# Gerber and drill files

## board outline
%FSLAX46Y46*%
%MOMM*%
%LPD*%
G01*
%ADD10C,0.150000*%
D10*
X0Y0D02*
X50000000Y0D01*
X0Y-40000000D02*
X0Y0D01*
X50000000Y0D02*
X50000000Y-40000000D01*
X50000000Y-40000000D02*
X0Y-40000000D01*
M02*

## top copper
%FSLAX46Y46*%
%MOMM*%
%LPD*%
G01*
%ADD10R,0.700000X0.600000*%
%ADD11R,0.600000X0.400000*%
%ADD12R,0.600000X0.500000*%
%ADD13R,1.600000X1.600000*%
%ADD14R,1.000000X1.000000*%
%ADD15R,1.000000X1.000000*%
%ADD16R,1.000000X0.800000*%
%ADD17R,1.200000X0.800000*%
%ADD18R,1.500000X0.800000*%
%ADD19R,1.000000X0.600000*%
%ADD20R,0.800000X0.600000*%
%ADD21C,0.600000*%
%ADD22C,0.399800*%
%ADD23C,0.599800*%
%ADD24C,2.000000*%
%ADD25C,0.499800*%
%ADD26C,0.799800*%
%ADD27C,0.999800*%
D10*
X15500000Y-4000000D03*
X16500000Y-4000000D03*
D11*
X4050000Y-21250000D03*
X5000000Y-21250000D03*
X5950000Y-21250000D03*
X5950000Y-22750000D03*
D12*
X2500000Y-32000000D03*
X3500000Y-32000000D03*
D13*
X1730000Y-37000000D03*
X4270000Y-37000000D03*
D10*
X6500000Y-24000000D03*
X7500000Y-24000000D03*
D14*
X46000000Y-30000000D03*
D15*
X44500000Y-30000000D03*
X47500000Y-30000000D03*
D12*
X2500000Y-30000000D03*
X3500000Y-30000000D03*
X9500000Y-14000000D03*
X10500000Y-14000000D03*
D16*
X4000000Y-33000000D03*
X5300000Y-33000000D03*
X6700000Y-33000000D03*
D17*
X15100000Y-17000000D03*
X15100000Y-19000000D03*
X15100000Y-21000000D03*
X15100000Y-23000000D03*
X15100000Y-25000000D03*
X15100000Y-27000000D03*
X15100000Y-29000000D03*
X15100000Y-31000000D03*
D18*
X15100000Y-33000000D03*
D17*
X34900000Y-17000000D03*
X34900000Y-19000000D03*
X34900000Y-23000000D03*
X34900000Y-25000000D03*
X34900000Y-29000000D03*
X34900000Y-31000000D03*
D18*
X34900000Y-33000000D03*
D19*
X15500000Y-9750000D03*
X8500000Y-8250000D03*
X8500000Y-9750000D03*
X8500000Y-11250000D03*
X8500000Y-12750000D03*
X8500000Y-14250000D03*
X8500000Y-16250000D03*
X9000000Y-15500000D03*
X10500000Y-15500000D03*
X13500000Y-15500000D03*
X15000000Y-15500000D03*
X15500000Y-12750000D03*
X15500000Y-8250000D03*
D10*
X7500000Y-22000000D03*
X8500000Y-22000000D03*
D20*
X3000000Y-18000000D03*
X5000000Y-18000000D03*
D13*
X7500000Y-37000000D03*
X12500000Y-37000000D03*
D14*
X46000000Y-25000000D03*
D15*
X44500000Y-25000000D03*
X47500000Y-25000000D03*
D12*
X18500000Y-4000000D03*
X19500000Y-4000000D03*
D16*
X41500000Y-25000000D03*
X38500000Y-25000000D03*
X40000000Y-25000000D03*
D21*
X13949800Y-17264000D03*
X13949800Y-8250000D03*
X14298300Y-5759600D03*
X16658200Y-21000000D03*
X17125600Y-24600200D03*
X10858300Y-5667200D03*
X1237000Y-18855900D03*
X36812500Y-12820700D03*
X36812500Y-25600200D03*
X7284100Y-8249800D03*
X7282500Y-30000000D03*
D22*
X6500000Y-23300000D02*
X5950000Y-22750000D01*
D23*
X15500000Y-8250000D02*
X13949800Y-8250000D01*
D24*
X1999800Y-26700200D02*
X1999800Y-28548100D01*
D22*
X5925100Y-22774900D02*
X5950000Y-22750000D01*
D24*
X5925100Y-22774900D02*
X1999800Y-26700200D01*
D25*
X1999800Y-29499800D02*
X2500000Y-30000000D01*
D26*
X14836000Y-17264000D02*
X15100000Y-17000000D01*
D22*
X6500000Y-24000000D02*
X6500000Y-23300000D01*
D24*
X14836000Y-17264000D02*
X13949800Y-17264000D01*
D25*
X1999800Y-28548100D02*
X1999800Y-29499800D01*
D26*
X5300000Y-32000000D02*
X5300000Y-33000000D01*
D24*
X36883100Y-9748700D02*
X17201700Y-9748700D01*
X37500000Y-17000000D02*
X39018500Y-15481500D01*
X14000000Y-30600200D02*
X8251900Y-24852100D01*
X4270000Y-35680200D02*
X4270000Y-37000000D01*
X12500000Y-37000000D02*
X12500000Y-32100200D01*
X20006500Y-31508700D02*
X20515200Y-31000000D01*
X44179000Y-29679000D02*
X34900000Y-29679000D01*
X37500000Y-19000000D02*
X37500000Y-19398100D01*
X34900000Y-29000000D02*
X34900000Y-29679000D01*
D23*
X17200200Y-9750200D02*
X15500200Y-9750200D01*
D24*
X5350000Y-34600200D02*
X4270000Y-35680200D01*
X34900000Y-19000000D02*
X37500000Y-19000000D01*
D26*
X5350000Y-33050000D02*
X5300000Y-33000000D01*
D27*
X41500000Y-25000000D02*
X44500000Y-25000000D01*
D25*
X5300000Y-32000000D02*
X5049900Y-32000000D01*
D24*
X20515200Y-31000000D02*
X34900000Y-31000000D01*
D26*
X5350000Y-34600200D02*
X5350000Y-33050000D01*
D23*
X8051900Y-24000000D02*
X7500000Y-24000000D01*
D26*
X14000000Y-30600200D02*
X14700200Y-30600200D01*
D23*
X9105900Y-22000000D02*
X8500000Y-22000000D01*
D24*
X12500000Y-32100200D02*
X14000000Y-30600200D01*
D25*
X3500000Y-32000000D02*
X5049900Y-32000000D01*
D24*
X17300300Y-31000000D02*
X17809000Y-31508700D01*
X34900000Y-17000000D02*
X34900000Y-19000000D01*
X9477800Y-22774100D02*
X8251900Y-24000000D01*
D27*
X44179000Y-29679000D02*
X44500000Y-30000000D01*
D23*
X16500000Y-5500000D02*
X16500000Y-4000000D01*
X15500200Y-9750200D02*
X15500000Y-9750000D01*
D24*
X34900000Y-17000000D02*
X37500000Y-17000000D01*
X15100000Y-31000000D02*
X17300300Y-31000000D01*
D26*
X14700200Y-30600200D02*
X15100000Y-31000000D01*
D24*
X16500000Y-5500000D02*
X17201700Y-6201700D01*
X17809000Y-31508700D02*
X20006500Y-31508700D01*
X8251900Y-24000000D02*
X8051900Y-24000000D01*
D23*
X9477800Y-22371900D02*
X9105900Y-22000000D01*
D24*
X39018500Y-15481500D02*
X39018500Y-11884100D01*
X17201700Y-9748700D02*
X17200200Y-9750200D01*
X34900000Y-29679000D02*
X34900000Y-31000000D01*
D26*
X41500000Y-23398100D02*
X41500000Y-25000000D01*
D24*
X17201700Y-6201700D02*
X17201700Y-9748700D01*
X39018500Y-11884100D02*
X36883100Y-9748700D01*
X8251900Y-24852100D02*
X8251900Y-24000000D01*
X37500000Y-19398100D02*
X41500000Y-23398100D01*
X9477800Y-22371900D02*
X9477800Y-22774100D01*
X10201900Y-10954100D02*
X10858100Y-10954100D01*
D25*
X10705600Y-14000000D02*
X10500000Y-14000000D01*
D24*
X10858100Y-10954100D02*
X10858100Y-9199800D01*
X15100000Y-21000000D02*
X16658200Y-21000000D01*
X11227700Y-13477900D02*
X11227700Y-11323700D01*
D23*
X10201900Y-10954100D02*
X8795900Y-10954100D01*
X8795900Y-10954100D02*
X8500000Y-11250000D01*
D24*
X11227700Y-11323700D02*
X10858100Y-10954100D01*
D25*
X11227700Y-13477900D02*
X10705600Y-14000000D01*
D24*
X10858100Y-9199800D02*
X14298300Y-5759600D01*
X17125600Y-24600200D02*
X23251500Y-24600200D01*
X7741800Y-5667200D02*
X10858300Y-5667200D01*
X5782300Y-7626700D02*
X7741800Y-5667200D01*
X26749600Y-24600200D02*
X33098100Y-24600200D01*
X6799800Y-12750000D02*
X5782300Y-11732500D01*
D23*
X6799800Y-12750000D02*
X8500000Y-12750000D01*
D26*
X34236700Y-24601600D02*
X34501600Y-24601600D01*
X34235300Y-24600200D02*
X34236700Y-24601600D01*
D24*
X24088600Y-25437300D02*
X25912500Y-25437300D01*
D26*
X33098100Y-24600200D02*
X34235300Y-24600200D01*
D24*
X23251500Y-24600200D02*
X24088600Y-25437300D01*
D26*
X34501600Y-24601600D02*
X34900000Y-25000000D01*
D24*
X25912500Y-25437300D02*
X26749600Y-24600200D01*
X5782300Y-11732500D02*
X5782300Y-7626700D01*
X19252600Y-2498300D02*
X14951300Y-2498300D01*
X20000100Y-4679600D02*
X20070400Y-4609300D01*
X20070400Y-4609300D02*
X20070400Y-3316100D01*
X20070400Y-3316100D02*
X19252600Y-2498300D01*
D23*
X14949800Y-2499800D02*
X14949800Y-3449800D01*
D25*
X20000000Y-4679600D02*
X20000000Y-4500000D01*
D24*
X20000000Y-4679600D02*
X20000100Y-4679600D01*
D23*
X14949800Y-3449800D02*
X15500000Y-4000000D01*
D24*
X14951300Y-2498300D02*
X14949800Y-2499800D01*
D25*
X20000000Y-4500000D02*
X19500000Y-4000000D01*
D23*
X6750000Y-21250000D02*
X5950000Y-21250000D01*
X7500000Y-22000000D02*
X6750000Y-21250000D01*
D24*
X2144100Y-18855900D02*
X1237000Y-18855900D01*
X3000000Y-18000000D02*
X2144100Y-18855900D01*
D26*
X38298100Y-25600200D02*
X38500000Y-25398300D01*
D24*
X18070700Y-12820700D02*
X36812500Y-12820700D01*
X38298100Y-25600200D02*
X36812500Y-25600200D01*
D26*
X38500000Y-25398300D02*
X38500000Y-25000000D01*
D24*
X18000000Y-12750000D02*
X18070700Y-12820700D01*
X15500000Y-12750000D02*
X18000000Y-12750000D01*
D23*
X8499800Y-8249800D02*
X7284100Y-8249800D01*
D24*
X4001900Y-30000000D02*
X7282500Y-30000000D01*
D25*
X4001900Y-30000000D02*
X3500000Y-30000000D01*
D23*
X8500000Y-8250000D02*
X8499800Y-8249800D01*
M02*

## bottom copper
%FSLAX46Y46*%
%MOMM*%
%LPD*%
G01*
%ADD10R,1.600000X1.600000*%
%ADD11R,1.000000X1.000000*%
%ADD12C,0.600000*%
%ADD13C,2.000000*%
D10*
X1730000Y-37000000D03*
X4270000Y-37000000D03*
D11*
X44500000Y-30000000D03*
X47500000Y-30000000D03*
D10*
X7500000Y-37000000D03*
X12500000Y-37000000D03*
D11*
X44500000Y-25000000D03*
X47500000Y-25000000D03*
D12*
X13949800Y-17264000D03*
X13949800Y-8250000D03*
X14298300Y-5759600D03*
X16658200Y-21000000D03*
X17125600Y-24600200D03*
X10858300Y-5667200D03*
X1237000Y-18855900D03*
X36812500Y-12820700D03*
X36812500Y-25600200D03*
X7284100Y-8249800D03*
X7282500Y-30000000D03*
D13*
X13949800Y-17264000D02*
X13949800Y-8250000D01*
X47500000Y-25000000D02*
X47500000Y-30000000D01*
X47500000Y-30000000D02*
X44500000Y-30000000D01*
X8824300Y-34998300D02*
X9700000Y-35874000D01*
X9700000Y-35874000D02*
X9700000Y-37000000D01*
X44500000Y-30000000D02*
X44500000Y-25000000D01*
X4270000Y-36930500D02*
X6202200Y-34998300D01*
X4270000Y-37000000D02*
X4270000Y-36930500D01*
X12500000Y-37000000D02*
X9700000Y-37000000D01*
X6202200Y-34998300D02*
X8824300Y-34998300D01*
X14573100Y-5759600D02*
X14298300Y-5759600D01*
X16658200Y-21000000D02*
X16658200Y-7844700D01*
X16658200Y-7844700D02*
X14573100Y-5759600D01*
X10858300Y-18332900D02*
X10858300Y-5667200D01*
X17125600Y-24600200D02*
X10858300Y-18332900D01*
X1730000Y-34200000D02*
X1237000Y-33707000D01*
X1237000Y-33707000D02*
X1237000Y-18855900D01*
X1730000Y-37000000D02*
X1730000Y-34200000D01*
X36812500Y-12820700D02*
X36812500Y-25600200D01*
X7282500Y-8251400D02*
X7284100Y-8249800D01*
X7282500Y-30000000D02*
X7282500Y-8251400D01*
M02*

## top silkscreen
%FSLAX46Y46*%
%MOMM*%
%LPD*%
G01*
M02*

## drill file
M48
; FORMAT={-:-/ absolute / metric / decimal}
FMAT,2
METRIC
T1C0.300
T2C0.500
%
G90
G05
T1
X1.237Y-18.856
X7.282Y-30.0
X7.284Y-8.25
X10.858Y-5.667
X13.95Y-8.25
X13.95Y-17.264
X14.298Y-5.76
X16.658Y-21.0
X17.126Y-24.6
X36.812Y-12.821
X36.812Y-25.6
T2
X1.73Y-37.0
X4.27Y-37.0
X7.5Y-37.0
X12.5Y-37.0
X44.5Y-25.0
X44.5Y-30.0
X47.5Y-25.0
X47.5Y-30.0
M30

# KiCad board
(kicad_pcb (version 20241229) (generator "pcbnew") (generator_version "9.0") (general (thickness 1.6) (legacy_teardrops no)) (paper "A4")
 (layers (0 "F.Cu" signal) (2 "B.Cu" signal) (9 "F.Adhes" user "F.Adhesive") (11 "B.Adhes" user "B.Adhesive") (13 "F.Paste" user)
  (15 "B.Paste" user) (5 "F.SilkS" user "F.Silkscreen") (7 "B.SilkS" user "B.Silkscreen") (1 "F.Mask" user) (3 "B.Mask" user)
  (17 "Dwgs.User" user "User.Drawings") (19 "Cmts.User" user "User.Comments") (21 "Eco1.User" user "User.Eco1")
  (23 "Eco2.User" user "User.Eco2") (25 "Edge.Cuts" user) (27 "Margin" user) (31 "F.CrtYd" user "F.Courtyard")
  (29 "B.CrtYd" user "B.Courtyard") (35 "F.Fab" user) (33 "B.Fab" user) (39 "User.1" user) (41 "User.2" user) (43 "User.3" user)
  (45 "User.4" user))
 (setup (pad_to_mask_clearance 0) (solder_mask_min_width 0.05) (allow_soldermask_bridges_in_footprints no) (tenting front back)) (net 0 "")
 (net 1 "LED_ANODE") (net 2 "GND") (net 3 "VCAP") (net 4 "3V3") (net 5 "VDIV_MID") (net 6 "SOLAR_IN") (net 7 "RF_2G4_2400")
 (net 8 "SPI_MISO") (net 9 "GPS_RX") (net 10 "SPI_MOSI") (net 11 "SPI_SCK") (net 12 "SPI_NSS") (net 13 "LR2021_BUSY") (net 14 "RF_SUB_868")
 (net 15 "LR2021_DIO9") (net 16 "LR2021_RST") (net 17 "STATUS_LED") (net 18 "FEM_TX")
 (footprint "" (layer "F.Cu") (at 16 4)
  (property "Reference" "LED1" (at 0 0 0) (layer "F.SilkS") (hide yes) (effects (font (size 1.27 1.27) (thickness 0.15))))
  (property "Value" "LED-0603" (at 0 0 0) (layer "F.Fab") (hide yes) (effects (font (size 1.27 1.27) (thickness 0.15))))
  (pad "A" smd rect (at -0.5 0) (size 0.7 0.6) (layers "F.Cu" "F.Mask") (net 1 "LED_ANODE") (thermal_bridge_angle 45))
  (pad "K" smd rect (at 0.5 0) (size 0.7 0.6) (layers "F.Cu" "F.Mask") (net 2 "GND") (thermal_bridge_angle 45)))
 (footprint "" (layer "F.Cu") (at 5 22)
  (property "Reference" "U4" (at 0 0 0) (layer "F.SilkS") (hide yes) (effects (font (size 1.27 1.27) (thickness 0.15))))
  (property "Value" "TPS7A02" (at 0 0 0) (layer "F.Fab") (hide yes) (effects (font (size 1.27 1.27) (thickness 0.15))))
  (pad "1" smd rect (at -0.95 -0.75) (size 0.6 0.4) (layers "F.Cu" "F.Mask") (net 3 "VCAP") (thermal_bridge_angle 45))
  (pad "2" smd rect (at 0 -0.75) (size 0.6 0.4) (layers "F.Cu" "F.Mask") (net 2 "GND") (thermal_bridge_angle 45))
  (pad "3" smd rect (at 0.95 -0.75) (size 0.6 0.4) (layers "F.Cu" "F.Mask") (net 3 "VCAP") (thermal_bridge_angle 45))
  (pad "4" smd rect (at 0.95 0.75) (size 0.6 0.4) (layers "F.Cu" "F.Mask") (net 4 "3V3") (thermal_bridge_angle 45)))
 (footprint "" (layer "F.Cu") (at 3 32)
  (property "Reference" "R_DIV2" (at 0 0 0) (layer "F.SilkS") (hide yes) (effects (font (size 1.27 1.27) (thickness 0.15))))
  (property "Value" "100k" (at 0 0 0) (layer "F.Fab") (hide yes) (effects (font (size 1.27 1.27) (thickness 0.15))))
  (pad "1" smd rect (at -0.5 0) (size 0.6 0.5) (layers "F.Cu" "F.Mask") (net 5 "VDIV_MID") (thermal_bridge_angle 45))
  (pad "2" smd rect (at 0.5 0) (size 0.6 0.5) (layers "F.Cu" "F.Mask") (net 2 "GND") (thermal_bridge_angle 45)))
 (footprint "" (layer "F.Cu") (at 3 37)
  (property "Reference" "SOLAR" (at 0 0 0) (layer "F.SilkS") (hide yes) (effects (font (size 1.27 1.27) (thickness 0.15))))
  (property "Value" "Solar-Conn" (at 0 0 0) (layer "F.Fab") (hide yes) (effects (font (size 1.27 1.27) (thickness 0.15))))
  (pad "1" thru_hole rect (at -1.27 0) (size 1.6 1.6) (drill 0.5) (layers "*.Cu" "*.Mask") (remove_unused_layers no) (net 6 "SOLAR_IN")
   (thermal_bridge_angle 45))
  (pad "2" thru_hole rect (at 1.27 0) (size 1.6 1.6) (drill 0.5) (layers "*.Cu" "*.Mask") (remove_unused_layers no) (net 2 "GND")
   (thermal_bridge_angle 45)))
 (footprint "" (layer "F.Cu") (at 7 24)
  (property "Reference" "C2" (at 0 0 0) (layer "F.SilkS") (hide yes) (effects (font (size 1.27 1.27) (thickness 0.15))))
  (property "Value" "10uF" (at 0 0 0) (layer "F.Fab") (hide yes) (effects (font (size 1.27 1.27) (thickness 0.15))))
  (pad "1" smd rect (at -0.5 0) (size 0.7 0.6) (layers "F.Cu" "F.Mask") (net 4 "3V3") (thermal_bridge_angle 45))
  (pad "2" smd rect (at 0.5 0) (size 0.7 0.6) (layers "F.Cu" "F.Mask") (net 2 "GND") (thermal_bridge_angle 45)))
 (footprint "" (layer "F.Cu") (at 46 30)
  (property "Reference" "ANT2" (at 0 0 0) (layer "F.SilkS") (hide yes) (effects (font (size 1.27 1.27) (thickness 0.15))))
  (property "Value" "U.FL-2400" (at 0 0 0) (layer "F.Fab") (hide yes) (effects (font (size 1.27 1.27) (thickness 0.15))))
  (pad "1" smd rect (at 0 0) (size 1 1) (layers "F.Cu" "F.Mask") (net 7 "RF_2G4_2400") (thermal_bridge_angle 45))
  (pad "2" thru_hole rect (at -1.5 0) (size 1 1) (drill 0.5) (layers "*.Cu" "*.Mask") (remove_unused_layers no) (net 2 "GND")
   (thermal_bridge_angle 45))
  (pad "3" thru_hole rect (at 1.5 0) (size 1 1) (drill 0.5) (layers "*.Cu" "*.Mask") (remove_unused_layers no) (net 2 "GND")
   (thermal_bridge_angle 45)))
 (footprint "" (layer "F.Cu") (at 3 30)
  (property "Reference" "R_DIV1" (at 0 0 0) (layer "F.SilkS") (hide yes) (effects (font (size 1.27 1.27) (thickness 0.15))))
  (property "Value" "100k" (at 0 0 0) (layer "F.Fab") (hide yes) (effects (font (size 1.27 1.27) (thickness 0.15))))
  (pad "1" smd rect (at -0.5 0) (size 0.6 0.5) (layers "F.Cu" "F.Mask") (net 4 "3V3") (thermal_bridge_angle 45))
  (pad "2" smd rect (at 0.5 0) (size 0.6 0.5) (layers "F.Cu" "F.Mask") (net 5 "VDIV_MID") (thermal_bridge_angle 45)))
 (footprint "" (layer "F.Cu") (at 10 14)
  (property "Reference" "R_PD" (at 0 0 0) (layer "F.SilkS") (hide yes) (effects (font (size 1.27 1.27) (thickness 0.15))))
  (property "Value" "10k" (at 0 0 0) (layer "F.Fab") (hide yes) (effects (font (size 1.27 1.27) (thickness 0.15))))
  (pad "1" smd rect (at -0.5 0) (size 0.6 0.5) (layers "F.Cu" "F.Mask") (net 2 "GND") (thermal_bridge_angle 45))
  (pad "2" smd rect (at 0.5 0) (size 0.6 0.5) (layers "F.Cu" "F.Mask") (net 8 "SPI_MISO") (thermal_bridge_angle 45)))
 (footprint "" (layer "F.Cu") (at 6 33)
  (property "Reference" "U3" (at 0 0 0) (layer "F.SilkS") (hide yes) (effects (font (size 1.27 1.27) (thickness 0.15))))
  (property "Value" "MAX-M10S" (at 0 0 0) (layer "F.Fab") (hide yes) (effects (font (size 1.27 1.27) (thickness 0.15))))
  (pad "1" smd rect (at -2 0) (size 1 0.8) (layers "F.Cu" "F.Mask") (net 4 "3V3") (thermal_bridge_angle 45))
  (pad "2" smd rect (at -0.7 0) (size 1 0.8) (layers "F.Cu" "F.Mask") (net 2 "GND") (thermal_bridge_angle 45))
  (pad "3" smd rect (at 0.7 0) (size 1 0.8) (layers "F.Cu" "F.Mask") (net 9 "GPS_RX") (thermal_bridge_angle 45)))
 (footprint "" (layer "F.Cu") (at 25 25)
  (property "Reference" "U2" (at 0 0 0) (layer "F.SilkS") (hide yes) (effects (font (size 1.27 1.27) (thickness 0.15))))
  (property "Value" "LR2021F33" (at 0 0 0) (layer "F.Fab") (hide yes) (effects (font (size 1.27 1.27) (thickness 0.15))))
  (pad "1" smd rect (at -9.9 -8) (size 1.2 0.8) (layers "F.Cu" "F.Mask") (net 4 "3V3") (thermal_bridge_angle 45))
  (pad "2" smd rect (at -9.9 -6) (size 1.2 0.8) (layers "F.Cu" "F.Mask") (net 2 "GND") (thermal_bridge_angle 45))
  (pad "3" smd rect (at -9.9 -4) (size 1.2 0.8) (layers "F.Cu" "F.Mask") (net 8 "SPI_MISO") (thermal_bridge_angle 45))
  (pad "4" smd rect (at -9.9 -2) (size 1.2 0.8) (layers "F.Cu" "F.Mask") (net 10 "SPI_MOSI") (thermal_bridge_angle 45))
  (pad "5" smd rect (at -9.9 0) (size 1.2 0.8) (layers "F.Cu" "F.Mask") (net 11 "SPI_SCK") (thermal_bridge_angle 45))
  (pad "6" smd rect (at -9.9 2) (size 1.2 0.8) (layers "F.Cu" "F.Mask") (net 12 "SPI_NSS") (thermal_bridge_angle 45))
  (pad "7" smd rect (at -9.9 4) (size 1.2 0.8) (layers "F.Cu" "F.Mask") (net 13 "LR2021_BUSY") (thermal_bridge_angle 45))
  (pad "8" smd rect (at -9.9 6) (size 1.2 0.8) (layers "F.Cu" "F.Mask") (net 2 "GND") (thermal_bridge_angle 45))
  (pad "9" smd rect (at -9.9 8) (size 1.5 0.8) (layers "F.Cu" "F.Mask") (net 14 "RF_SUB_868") (thermal_bridge_angle 45))
  (pad "10" smd rect (at 9.9 -8) (size 1.2 0.8) (layers "F.Cu" "F.Mask") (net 2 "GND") (thermal_bridge_angle 45))
  (pad "11" smd rect (at 9.9 -6) (size 1.2 0.8) (layers "F.Cu" "F.Mask") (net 2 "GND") (thermal_bridge_angle 45))
  (pad "13" smd rect (at 9.9 -2) (size 1.2 0.8) (layers "F.Cu" "F.Mask") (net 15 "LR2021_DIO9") (thermal_bridge_angle 45))
  (pad "14" smd rect (at 9.9 0) (size 1.2 0.8) (layers "F.Cu" "F.Mask") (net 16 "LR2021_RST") (thermal_bridge_angle 45))
  (pad "16" smd rect (at 9.9 4) (size 1.2 0.8) (layers "F.Cu" "F.Mask") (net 2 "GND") (thermal_bridge_angle 45))
  (pad "17" smd rect (at 9.9 6) (size 1.2 0.8) (layers "F.Cu" "F.Mask") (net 2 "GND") (thermal_bridge_angle 45))
  (pad "18" smd rect (at 9.9 8) (size 1.5 0.8) (layers "F.Cu" "F.Mask") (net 7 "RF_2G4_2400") (thermal_bridge_angle 45)))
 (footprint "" (layer "F.Cu") (at 12 12)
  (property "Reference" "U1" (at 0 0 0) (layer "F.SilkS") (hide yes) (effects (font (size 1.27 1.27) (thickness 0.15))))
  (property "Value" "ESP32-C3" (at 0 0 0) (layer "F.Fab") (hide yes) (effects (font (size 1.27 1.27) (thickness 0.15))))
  (pad "GND" smd rect (at 3.5 -2.25) (size 1 0.6) (layers "F.Cu" "F.Mask") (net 2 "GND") (thermal_bridge_angle 45))
  (pad "GPIO0" smd rect (at -3.5 -3.75) (size 1 0.6) (layers "F.Cu" "F.Mask") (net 5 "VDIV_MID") (thermal_bridge_angle 45))
  (pad "GPIO1" smd rect (at -3.5 -2.25) (size 1 0.6) (layers "F.Cu" "F.Mask") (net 9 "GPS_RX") (thermal_bridge_angle 45))
  (pad "GPIO2" smd rect (at -3.5 -0.75) (size 1 0.6) (layers "F.Cu" "F.Mask") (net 8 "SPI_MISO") (thermal_bridge_angle 45))
  (pad "GPIO3" smd rect (at -3.5 0.75) (size 1 0.6) (layers "F.Cu" "F.Mask") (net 16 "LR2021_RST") (thermal_bridge_angle 45))
  (pad "GPIO4" smd rect (at -3.5 2.25) (size 1 0.6) (layers "F.Cu" "F.Mask") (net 13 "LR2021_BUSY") (thermal_bridge_angle 45))
  (pad "GPIO5" smd rect (at -3.5 4.25) (size 1 0.6) (layers "F.Cu" "F.Mask") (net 15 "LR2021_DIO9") (thermal_bridge_angle 45))
  (pad "GPIO6" smd rect (at -3 3.5) (size 1 0.6) (layers "F.Cu" "F.Mask") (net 11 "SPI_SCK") (thermal_bridge_angle 45))
  (pad "GPIO7" smd rect (at -1.5 3.5) (size 1 0.6) (layers "F.Cu" "F.Mask") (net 10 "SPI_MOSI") (thermal_bridge_angle 45))
  (pad "GPIO9" smd rect (at 1.5 3.5) (size 1 0.6) (layers "F.Cu" "F.Mask") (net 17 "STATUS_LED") (thermal_bridge_angle 45))
  (pad "GPIO10" smd rect (at 3 3.5) (size 1 0.6) (layers "F.Cu" "F.Mask") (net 12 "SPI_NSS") (thermal_bridge_angle 45))
  (pad "GPIO19" smd rect (at 3.5 0.75) (size 1 0.6) (layers "F.Cu" "F.Mask") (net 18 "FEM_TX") (thermal_bridge_angle 45))
  (pad "VCC" smd rect (at 3.5 -3.75) (size 1 0.6) (layers "F.Cu" "F.Mask") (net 4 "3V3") (thermal_bridge_angle 45)))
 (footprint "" (layer "F.Cu") (at 8 22)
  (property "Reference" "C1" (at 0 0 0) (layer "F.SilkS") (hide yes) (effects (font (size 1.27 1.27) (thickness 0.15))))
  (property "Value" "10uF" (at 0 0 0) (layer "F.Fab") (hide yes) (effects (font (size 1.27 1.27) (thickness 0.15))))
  (pad "1" smd rect (at -0.5 0) (size 0.7 0.6) (layers "F.Cu" "F.Mask") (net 3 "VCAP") (thermal_bridge_angle 45))
  (pad "2" smd rect (at 0.5 0) (size 0.7 0.6) (layers "F.Cu" "F.Mask") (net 2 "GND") (thermal_bridge_angle 45)))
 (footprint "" (layer "F.Cu") (at 4 18)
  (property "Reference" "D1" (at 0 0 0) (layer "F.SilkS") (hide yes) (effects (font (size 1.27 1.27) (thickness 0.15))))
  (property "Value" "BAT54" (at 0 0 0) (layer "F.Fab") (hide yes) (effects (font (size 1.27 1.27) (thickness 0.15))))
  (pad "A" smd rect (at -1 0) (size 0.8 0.6) (layers "F.Cu" "F.Mask") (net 6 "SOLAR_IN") (thermal_bridge_angle 45))
  (pad "K" smd rect (at 1 0) (size 0.8 0.6) (layers "F.Cu" "F.Mask") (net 3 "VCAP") (thermal_bridge_angle 45)))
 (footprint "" (layer "F.Cu") (at 10 37)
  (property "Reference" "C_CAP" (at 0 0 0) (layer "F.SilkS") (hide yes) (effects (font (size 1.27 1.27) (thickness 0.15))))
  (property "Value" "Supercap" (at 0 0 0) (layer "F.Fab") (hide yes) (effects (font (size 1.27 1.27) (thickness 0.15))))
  (pad "1" thru_hole rect (at -2.5 0) (size 1.6 1.6) (drill 0.5) (layers "*.Cu" "*.Mask") (remove_unused_layers no) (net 3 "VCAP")
   (thermal_bridge_angle 45))
  (pad "2" thru_hole rect (at 2.5 0) (size 1.6 1.6) (drill 0.5) (layers "*.Cu" "*.Mask") (remove_unused_layers no) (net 2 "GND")
   (thermal_bridge_angle 45)))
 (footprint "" (layer "F.Cu") (at 46 25)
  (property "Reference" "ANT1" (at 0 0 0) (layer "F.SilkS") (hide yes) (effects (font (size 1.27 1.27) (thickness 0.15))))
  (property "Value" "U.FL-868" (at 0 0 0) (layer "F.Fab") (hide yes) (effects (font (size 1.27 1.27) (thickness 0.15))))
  (pad "1" smd rect (at 0 0) (size 1 1) (layers "F.Cu" "F.Mask") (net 14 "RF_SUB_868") (thermal_bridge_angle 45))
  (pad "2" thru_hole rect (at -1.5 0) (size 1 1) (drill 0.5) (layers "*.Cu" "*.Mask") (remove_unused_layers no) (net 2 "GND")
   (thermal_bridge_angle 45))
  (pad "3" thru_hole rect (at 1.5 0) (size 1 1) (drill 0.5) (layers "*.Cu" "*.Mask") (remove_unused_layers no) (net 2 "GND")
   (thermal_bridge_angle 45)))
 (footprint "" (layer "F.Cu") (at 19 4)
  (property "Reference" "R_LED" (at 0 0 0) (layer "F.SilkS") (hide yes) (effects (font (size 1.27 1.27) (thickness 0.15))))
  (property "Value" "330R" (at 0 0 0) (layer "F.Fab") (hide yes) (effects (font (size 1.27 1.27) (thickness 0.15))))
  (pad "1" smd rect (at -0.5 0) (size 0.6 0.5) (layers "F.Cu" "F.Mask") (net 17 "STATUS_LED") (thermal_bridge_angle 45))
  (pad "2" smd rect (at 0.5 0) (size 0.6 0.5) (layers "F.Cu" "F.Mask") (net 1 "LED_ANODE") (thermal_bridge_angle 45)))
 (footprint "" (layer "F.Cu") (at 40 25)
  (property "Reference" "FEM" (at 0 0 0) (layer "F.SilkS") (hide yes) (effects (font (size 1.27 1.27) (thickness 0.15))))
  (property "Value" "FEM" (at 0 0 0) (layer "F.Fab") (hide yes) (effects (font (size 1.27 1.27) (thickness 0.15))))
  (pad "GND" smd rect (at 1.5 0) (size 1 0.8) (layers "F.Cu" "F.Mask") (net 2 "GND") (thermal_bridge_angle 45))
  (pad "TX" smd rect (at -1.5 0) (size 1 0.8) (layers "F.Cu" "F.Mask") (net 18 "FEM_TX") (thermal_bridge_angle 45))
  (pad "VCC" smd rect (at 0 0) (size 1 0.8) (layers "F.Cu" "F.Mask") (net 4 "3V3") (thermal_bridge_angle 45)))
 (gr_line (start 0 0) (end 50 0) (stroke (width 0.15) (type default)) (layer "Edge.Cuts"))
 (gr_line (start 0 40) (end 0 0) (stroke (width 0.15) (type default)) (layer "Edge.Cuts"))
 (gr_line (start 50 0) (end 50 40) (stroke (width 0.15) (type default)) (layer "Edge.Cuts"))
 (gr_line (start 50 40) (end 0 40) (stroke (width 0.15) (type default)) (layer "Edge.Cuts"))
 (segment (start 6.5 23.3) (end 5.95 22.75) (width 0.3998) (layer "F.Cu") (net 4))
 (segment (start 15.5 8.25) (end 13.9498 8.25) (width 0.5998) (layer "F.Cu") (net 4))
 (segment (start 1.9998 26.7002) (end 1.9998 28.5481) (width 2) (layer "F.Cu") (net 4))
 (segment (start 5.9251 22.7749) (end 5.95 22.75) (width 0.3998) (layer "F.Cu") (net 4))
 (segment (start 5.9251 22.7749) (end 1.9998 26.7002) (width 2) (layer "F.Cu") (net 4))
 (segment (start 1.9998 29.4998) (end 2.5 30) (width 0.4998) (layer "F.Cu") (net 4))
 (segment (start 14.836 17.264) (end 15.1 17) (width 0.7998) (layer "F.Cu") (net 4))
 (segment (start 6.5 24) (end 6.5 23.3) (width 0.3998) (layer "F.Cu") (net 4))
 (segment (start 14.836 17.264) (end 13.9498 17.264) (width 2) (layer "F.Cu") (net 4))
 (segment (start 1.9998 28.5481) (end 1.9998 29.4998) (width 0.4998) (layer "F.Cu") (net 4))
 (via (at 13.9498 17.264) (size 0.6) (drill 0.3) (layers "F.Cu" "B.Cu") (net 4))
 (via (at 13.9498 8.25) (size 0.6) (drill 0.3) (layers "F.Cu" "B.Cu") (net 4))
 (segment (start 13.9498 17.264) (end 13.9498 8.25) (width 2) (layer "B.Cu") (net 4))
 (segment (start 5.3 32) (end 5.3 33) (width 0.7998) (layer "F.Cu") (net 2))
 (segment (start 36.8831 9.7487) (end 17.2017 9.7487) (width 2) (layer "F.Cu") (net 2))
 (segment (start 37.5 17) (end 39.0185 15.4815) (width 2) (layer "F.Cu") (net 2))
 (segment (start 14 30.6002) (end 8.2519 24.8521) (width 2) (layer "F.Cu") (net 2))
 (segment (start 4.27 35.6802) (end 4.27 37) (width 2) (layer "F.Cu") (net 2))
 (segment (start 12.5 37) (end 12.5 32.1002) (width 2) (layer "F.Cu") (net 2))
 (segment (start 20.0065 31.5087) (end 20.5152 31) (width 2) (layer "F.Cu") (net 2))
 (segment (start 44.179 29.679) (end 34.9 29.679) (width 2) (layer "F.Cu") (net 2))
 (segment (start 37.5 19) (end 37.5 19.3981) (width 2) (layer "F.Cu") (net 2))
 (segment (start 34.9 29) (end 34.9 29.679) (width 2) (layer "F.Cu") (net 2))
 (segment (start 17.2002 9.7502) (end 15.5002 9.7502) (width 0.5998) (layer "F.Cu") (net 2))
 (segment (start 5.35 34.6002) (end 4.27 35.6802) (width 2) (layer "F.Cu") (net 2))
 (segment (start 34.9 19) (end 37.5 19) (width 2) (layer "F.Cu") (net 2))
 (segment (start 5.35 33.05) (end 5.3 33) (width 0.7998) (layer "F.Cu") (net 2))
 (segment (start 41.5 25) (end 44.5 25) (width 0.9998) (layer "F.Cu") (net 2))
 (segment (start 5.3 32) (end 5.0499 32) (width 0.4998) (layer "F.Cu") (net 2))
 (segment (start 20.5152 31) (end 34.9 31) (width 2) (layer "F.Cu") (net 2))
 (segment (start 5.35 34.6002) (end 5.35 33.05) (width 0.7998) (layer "F.Cu") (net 2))
 (segment (start 8.0519 24) (end 7.5 24) (width 0.5998) (layer "F.Cu") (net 2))
 (segment (start 14 30.6002) (end 14.7002 30.6002) (width 0.7998) (layer "F.Cu") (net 2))
 (segment (start 9.1059 22) (end 8.5 22) (width 0.5998) (layer "F.Cu") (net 2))
 (segment (start 12.5 32.1002) (end 14 30.6002) (width 2) (layer "F.Cu") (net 2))
 (segment (start 3.5 32) (end 5.0499 32) (width 0.4998) (layer "F.Cu") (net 2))
 (segment (start 17.3003 31) (end 17.809 31.5087) (width 2) (layer "F.Cu") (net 2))
 (segment (start 34.9 17) (end 34.9 19) (width 2) (layer "F.Cu") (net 2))
 (segment (start 9.4778 22.7741) (end 8.2519 24) (width 2) (layer "F.Cu") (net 2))
 (segment (start 44.179 29.679) (end 44.5 30) (width 0.9998) (layer "F.Cu") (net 2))
 (segment (start 16.5 5.5) (end 16.5 4) (width 0.5998) (layer "F.Cu") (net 2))
 (segment (start 15.5002 9.7502) (end 15.5 9.75) (width 0.5998) (layer "F.Cu") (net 2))
 (segment (start 34.9 17) (end 37.5 17) (width 2) (layer "F.Cu") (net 2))
 (segment (start 15.1 31) (end 17.3003 31) (width 2) (layer "F.Cu") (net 2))
 (segment (start 14.7002 30.6002) (end 15.1 31) (width 0.7998) (layer "F.Cu") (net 2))
 (segment (start 16.5 5.5) (end 17.2017 6.2017) (width 2) (layer "F.Cu") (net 2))
 (segment (start 17.809 31.5087) (end 20.0065 31.5087) (width 2) (layer "F.Cu") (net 2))
 (segment (start 8.2519 24) (end 8.0519 24) (width 2) (layer "F.Cu") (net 2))
 (segment (start 9.4778 22.3719) (end 9.1059 22) (width 0.5998) (layer "F.Cu") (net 2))
 (segment (start 39.0185 15.4815) (end 39.0185 11.8841) (width 2) (layer "F.Cu") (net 2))
 (segment (start 17.2017 9.7487) (end 17.2002 9.7502) (width 2) (layer "F.Cu") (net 2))
 (segment (start 34.9 29.679) (end 34.9 31) (width 2) (layer "F.Cu") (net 2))
 (segment (start 41.5 23.3981) (end 41.5 25) (width 0.7998) (layer "F.Cu") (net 2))
 (segment (start 17.2017 6.2017) (end 17.2017 9.7487) (width 2) (layer "F.Cu") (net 2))
 (segment (start 39.0185 11.8841) (end 36.8831 9.7487) (width 2) (layer "F.Cu") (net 2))
 (segment (start 8.2519 24.8521) (end 8.2519 24) (width 2) (layer "F.Cu") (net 2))
 (segment (start 37.5 19.3981) (end 41.5 23.3981) (width 2) (layer "F.Cu") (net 2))
 (segment (start 9.4778 22.3719) (end 9.4778 22.7741) (width 2) (layer "F.Cu") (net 2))
 (segment (start 47.5 25) (end 47.5 30) (width 2) (layer "B.Cu") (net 2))
 (segment (start 47.5 30) (end 44.5 30) (width 2) (layer "B.Cu") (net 2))
 (segment (start 8.8243 34.9983) (end 9.7 35.874) (width 2) (layer "B.Cu") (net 2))
 (segment (start 9.7 35.874) (end 9.7 37) (width 2) (layer "B.Cu") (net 2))
 (segment (start 44.5 30) (end 44.5 25) (width 2) (layer "B.Cu") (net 2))
 (segment (start 4.27 36.9305) (end 6.2022 34.9983) (width 2) (layer "B.Cu") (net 2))
 (segment (start 4.27 37) (end 4.27 36.9305) (width 2) (layer "B.Cu") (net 2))
 (segment (start 12.5 37) (end 9.7 37) (width 2) (layer "B.Cu") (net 2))
 (segment (start 6.2022 34.9983) (end 8.8243 34.9983) (width 2) (layer "B.Cu") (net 2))
 (segment (start 10.2019 10.9541) (end 10.8581 10.9541) (width 2) (layer "F.Cu") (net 8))
 (segment (start 10.7056 14) (end 10.5 14) (width 0.4998) (layer "F.Cu") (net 8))
 (segment (start 10.8581 10.9541) (end 10.8581 9.1998) (width 2) (layer "F.Cu") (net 8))
 (segment (start 15.1 21) (end 16.6582 21) (width 2) (layer "F.Cu") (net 8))
 (segment (start 11.2277 13.4779) (end 11.2277 11.3237) (width 2) (layer "F.Cu") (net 8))
 (segment (start 10.2019 10.9541) (end 8.7959 10.9541) (width 0.5998) (layer "F.Cu") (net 8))
 (segment (start 8.7959 10.9541) (end 8.5 11.25) (width 0.5998) (layer "F.Cu") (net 8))
 (segment (start 11.2277 11.3237) (end 10.8581 10.9541) (width 2) (layer "F.Cu") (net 8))
 (segment (start 11.2277 13.4779) (end 10.7056 14) (width 0.4998) (layer "F.Cu") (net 8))
 (segment (start 10.8581 9.1998) (end 14.2983 5.7596) (width 2) (layer "F.Cu") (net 8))
 (via (at 14.2983 5.7596) (size 0.6) (drill 0.3) (layers "F.Cu" "B.Cu") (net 8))
 (via (at 16.6582 21) (size 0.6) (drill 0.3) (layers "F.Cu" "B.Cu") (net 8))
 (segment (start 14.5731 5.7596) (end 14.2983 5.7596) (width 2) (layer "B.Cu") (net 8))
 (segment (start 16.6582 21) (end 16.6582 7.8447) (width 2) (layer "B.Cu") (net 8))
 (segment (start 16.6582 7.8447) (end 14.5731 5.7596) (width 2) (layer "B.Cu") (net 8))
 (segment (start 17.1256 24.6002) (end 23.2515 24.6002) (width 2) (layer "F.Cu") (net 16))
 (segment (start 7.7418 5.6672) (end 10.8583 5.6672) (width 2) (layer "F.Cu") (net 16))
 (segment (start 5.7823 7.6267) (end 7.7418 5.6672) (width 2) (layer "F.Cu") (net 16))
 (segment (start 26.7496 24.6002) (end 33.0981 24.6002) (width 2) (layer "F.Cu") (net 16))
 (segment (start 6.7998 12.75) (end 5.7823 11.7325) (width 2) (layer "F.Cu") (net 16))
 (segment (start 6.7998 12.75) (end 8.5 12.75) (width 0.5998) (layer "F.Cu") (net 16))
 (segment (start 34.2367 24.6016) (end 34.5016 24.6016) (width 0.7998) (layer "F.Cu") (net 16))
 (segment (start 34.2353 24.6002) (end 34.2367 24.6016) (width 0.7998) (layer "F.Cu") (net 16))
 (segment (start 24.0886 25.4373) (end 25.9125 25.4373) (width 2) (layer "F.Cu") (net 16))
 (segment (start 33.0981 24.6002) (end 34.2353 24.6002) (width 0.7998) (layer "F.Cu") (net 16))
 (segment (start 23.2515 24.6002) (end 24.0886 25.4373) (width 2) (layer "F.Cu") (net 16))
 (segment (start 34.5016 24.6016) (end 34.9 25) (width 0.7998) (layer "F.Cu") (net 16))
 (segment (start 25.9125 25.4373) (end 26.7496 24.6002) (width 2) (layer "F.Cu") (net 16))
 (segment (start 5.7823 11.7325) (end 5.7823 7.6267) (width 2) (layer "F.Cu") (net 16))
 (via (at 17.1256 24.6002) (size 0.6) (drill 0.3) (layers "F.Cu" "B.Cu") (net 16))
 (via (at 10.8583 5.6672) (size 0.6) (drill 0.3) (layers "F.Cu" "B.Cu") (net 16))
 (segment (start 10.8583 18.3329) (end 10.8583 5.6672) (width 2) (layer "B.Cu") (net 16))
 (segment (start 17.1256 24.6002) (end 10.8583 18.3329) (width 2) (layer "B.Cu") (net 16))
 (segment (start 19.2526 2.4983) (end 14.9513 2.4983) (width 2) (layer "F.Cu") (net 1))
 (segment (start 20.0001 4.6796) (end 20.0704 4.6093) (width 2) (layer "F.Cu") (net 1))
 (segment (start 20.0704 4.6093) (end 20.0704 3.3161) (width 2) (layer "F.Cu") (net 1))
 (segment (start 20.0704 3.3161) (end 19.2526 2.4983) (width 2) (layer "F.Cu") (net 1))
 (segment (start 14.9498 2.4998) (end 14.9498 3.4498) (width 0.5998) (layer "F.Cu") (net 1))
 (segment (start 20 4.6796) (end 20 4.5) (width 0.4998) (layer "F.Cu") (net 1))
 (segment (start 20 4.6796) (end 20.0001 4.6796) (width 2) (layer "F.Cu") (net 1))
 (segment (start 14.9498 3.4498) (end 15.5 4) (width 0.5998) (layer "F.Cu") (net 1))
 (segment (start 14.9513 2.4983) (end 14.9498 2.4998) (width 2) (layer "F.Cu") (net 1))
 (segment (start 20 4.5) (end 19.5 4) (width 0.4998) (layer "F.Cu") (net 1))
 (segment (start 6.75 21.25) (end 5.95 21.25) (width 0.5998) (layer "F.Cu") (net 3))
 (segment (start 7.5 22) (end 6.75 21.25) (width 0.5998) (layer "F.Cu") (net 3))
 (segment (start 2.1441 18.8559) (end 1.237 18.8559) (width 2) (layer "F.Cu") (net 6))
 (segment (start 3 18) (end 2.1441 18.8559) (width 2) (layer "F.Cu") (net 6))
 (via (at 1.237 18.8559) (size 0.6) (drill 0.3) (layers "F.Cu" "B.Cu") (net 6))
 (segment (start 1.73 34.2) (end 1.237 33.707) (width 2) (layer "B.Cu") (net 6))
 (segment (start 1.237 33.707) (end 1.237 18.8559) (width 2) (layer "B.Cu") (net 6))
 (segment (start 1.73 37) (end 1.73 34.2) (width 2) (layer "B.Cu") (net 6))
 (segment (start 38.2981 25.6002) (end 38.5 25.3983) (width 0.7998) (layer "F.Cu") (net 18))
 (segment (start 18.0707 12.8207) (end 36.8125 12.8207) (width 2) (layer "F.Cu") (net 18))
 (segment (start 38.2981 25.6002) (end 36.8125 25.6002) (width 2) (layer "F.Cu") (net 18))
 (segment (start 38.5 25.3983) (end 38.5 25) (width 0.7998) (layer "F.Cu") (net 18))
 (segment (start 18 12.75) (end 18.0707 12.8207) (width 2) (layer "F.Cu") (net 18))
 (segment (start 15.5 12.75) (end 18 12.75) (width 2) (layer "F.Cu") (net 18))
 (via (at 36.8125 12.8207) (size 0.6) (drill 0.3) (layers "F.Cu" "B.Cu") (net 18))
 (via (at 36.8125 25.6002) (size 0.6) (drill 0.3) (layers "F.Cu" "B.Cu") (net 18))
 (segment (start 36.8125 12.8207) (end 36.8125 25.6002) (width 2) (layer "B.Cu") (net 18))
 (segment (start 8.4998 8.2498) (end 7.2841 8.2498) (width 0.5998) (layer "F.Cu") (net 5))
 (segment (start 4.0019 30) (end 7.2825 30) (width 2) (layer "F.Cu") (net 5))
 (segment (start 4.0019 30) (end 3.5 30) (width 0.4998) (layer "F.Cu") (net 5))
 (segment (start 8.5 8.25) (end 8.4998 8.2498) (width 0.5998) (layer "F.Cu") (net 5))
 (via (at 7.2841 8.2498) (size 0.6) (drill 0.3) (layers "F.Cu" "B.Cu") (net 5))
 (via (at 7.2825 30) (size 0.6) (drill 0.3) (layers "F.Cu" "B.Cu") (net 5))
 (segment (start 7.2825 8.2514) (end 7.2841 8.2498) (width 2) (layer "B.Cu") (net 5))
 (segment (start 7.2825 30) (end 7.2825 8.2514) (width 2) (layer "B.Cu") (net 5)))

